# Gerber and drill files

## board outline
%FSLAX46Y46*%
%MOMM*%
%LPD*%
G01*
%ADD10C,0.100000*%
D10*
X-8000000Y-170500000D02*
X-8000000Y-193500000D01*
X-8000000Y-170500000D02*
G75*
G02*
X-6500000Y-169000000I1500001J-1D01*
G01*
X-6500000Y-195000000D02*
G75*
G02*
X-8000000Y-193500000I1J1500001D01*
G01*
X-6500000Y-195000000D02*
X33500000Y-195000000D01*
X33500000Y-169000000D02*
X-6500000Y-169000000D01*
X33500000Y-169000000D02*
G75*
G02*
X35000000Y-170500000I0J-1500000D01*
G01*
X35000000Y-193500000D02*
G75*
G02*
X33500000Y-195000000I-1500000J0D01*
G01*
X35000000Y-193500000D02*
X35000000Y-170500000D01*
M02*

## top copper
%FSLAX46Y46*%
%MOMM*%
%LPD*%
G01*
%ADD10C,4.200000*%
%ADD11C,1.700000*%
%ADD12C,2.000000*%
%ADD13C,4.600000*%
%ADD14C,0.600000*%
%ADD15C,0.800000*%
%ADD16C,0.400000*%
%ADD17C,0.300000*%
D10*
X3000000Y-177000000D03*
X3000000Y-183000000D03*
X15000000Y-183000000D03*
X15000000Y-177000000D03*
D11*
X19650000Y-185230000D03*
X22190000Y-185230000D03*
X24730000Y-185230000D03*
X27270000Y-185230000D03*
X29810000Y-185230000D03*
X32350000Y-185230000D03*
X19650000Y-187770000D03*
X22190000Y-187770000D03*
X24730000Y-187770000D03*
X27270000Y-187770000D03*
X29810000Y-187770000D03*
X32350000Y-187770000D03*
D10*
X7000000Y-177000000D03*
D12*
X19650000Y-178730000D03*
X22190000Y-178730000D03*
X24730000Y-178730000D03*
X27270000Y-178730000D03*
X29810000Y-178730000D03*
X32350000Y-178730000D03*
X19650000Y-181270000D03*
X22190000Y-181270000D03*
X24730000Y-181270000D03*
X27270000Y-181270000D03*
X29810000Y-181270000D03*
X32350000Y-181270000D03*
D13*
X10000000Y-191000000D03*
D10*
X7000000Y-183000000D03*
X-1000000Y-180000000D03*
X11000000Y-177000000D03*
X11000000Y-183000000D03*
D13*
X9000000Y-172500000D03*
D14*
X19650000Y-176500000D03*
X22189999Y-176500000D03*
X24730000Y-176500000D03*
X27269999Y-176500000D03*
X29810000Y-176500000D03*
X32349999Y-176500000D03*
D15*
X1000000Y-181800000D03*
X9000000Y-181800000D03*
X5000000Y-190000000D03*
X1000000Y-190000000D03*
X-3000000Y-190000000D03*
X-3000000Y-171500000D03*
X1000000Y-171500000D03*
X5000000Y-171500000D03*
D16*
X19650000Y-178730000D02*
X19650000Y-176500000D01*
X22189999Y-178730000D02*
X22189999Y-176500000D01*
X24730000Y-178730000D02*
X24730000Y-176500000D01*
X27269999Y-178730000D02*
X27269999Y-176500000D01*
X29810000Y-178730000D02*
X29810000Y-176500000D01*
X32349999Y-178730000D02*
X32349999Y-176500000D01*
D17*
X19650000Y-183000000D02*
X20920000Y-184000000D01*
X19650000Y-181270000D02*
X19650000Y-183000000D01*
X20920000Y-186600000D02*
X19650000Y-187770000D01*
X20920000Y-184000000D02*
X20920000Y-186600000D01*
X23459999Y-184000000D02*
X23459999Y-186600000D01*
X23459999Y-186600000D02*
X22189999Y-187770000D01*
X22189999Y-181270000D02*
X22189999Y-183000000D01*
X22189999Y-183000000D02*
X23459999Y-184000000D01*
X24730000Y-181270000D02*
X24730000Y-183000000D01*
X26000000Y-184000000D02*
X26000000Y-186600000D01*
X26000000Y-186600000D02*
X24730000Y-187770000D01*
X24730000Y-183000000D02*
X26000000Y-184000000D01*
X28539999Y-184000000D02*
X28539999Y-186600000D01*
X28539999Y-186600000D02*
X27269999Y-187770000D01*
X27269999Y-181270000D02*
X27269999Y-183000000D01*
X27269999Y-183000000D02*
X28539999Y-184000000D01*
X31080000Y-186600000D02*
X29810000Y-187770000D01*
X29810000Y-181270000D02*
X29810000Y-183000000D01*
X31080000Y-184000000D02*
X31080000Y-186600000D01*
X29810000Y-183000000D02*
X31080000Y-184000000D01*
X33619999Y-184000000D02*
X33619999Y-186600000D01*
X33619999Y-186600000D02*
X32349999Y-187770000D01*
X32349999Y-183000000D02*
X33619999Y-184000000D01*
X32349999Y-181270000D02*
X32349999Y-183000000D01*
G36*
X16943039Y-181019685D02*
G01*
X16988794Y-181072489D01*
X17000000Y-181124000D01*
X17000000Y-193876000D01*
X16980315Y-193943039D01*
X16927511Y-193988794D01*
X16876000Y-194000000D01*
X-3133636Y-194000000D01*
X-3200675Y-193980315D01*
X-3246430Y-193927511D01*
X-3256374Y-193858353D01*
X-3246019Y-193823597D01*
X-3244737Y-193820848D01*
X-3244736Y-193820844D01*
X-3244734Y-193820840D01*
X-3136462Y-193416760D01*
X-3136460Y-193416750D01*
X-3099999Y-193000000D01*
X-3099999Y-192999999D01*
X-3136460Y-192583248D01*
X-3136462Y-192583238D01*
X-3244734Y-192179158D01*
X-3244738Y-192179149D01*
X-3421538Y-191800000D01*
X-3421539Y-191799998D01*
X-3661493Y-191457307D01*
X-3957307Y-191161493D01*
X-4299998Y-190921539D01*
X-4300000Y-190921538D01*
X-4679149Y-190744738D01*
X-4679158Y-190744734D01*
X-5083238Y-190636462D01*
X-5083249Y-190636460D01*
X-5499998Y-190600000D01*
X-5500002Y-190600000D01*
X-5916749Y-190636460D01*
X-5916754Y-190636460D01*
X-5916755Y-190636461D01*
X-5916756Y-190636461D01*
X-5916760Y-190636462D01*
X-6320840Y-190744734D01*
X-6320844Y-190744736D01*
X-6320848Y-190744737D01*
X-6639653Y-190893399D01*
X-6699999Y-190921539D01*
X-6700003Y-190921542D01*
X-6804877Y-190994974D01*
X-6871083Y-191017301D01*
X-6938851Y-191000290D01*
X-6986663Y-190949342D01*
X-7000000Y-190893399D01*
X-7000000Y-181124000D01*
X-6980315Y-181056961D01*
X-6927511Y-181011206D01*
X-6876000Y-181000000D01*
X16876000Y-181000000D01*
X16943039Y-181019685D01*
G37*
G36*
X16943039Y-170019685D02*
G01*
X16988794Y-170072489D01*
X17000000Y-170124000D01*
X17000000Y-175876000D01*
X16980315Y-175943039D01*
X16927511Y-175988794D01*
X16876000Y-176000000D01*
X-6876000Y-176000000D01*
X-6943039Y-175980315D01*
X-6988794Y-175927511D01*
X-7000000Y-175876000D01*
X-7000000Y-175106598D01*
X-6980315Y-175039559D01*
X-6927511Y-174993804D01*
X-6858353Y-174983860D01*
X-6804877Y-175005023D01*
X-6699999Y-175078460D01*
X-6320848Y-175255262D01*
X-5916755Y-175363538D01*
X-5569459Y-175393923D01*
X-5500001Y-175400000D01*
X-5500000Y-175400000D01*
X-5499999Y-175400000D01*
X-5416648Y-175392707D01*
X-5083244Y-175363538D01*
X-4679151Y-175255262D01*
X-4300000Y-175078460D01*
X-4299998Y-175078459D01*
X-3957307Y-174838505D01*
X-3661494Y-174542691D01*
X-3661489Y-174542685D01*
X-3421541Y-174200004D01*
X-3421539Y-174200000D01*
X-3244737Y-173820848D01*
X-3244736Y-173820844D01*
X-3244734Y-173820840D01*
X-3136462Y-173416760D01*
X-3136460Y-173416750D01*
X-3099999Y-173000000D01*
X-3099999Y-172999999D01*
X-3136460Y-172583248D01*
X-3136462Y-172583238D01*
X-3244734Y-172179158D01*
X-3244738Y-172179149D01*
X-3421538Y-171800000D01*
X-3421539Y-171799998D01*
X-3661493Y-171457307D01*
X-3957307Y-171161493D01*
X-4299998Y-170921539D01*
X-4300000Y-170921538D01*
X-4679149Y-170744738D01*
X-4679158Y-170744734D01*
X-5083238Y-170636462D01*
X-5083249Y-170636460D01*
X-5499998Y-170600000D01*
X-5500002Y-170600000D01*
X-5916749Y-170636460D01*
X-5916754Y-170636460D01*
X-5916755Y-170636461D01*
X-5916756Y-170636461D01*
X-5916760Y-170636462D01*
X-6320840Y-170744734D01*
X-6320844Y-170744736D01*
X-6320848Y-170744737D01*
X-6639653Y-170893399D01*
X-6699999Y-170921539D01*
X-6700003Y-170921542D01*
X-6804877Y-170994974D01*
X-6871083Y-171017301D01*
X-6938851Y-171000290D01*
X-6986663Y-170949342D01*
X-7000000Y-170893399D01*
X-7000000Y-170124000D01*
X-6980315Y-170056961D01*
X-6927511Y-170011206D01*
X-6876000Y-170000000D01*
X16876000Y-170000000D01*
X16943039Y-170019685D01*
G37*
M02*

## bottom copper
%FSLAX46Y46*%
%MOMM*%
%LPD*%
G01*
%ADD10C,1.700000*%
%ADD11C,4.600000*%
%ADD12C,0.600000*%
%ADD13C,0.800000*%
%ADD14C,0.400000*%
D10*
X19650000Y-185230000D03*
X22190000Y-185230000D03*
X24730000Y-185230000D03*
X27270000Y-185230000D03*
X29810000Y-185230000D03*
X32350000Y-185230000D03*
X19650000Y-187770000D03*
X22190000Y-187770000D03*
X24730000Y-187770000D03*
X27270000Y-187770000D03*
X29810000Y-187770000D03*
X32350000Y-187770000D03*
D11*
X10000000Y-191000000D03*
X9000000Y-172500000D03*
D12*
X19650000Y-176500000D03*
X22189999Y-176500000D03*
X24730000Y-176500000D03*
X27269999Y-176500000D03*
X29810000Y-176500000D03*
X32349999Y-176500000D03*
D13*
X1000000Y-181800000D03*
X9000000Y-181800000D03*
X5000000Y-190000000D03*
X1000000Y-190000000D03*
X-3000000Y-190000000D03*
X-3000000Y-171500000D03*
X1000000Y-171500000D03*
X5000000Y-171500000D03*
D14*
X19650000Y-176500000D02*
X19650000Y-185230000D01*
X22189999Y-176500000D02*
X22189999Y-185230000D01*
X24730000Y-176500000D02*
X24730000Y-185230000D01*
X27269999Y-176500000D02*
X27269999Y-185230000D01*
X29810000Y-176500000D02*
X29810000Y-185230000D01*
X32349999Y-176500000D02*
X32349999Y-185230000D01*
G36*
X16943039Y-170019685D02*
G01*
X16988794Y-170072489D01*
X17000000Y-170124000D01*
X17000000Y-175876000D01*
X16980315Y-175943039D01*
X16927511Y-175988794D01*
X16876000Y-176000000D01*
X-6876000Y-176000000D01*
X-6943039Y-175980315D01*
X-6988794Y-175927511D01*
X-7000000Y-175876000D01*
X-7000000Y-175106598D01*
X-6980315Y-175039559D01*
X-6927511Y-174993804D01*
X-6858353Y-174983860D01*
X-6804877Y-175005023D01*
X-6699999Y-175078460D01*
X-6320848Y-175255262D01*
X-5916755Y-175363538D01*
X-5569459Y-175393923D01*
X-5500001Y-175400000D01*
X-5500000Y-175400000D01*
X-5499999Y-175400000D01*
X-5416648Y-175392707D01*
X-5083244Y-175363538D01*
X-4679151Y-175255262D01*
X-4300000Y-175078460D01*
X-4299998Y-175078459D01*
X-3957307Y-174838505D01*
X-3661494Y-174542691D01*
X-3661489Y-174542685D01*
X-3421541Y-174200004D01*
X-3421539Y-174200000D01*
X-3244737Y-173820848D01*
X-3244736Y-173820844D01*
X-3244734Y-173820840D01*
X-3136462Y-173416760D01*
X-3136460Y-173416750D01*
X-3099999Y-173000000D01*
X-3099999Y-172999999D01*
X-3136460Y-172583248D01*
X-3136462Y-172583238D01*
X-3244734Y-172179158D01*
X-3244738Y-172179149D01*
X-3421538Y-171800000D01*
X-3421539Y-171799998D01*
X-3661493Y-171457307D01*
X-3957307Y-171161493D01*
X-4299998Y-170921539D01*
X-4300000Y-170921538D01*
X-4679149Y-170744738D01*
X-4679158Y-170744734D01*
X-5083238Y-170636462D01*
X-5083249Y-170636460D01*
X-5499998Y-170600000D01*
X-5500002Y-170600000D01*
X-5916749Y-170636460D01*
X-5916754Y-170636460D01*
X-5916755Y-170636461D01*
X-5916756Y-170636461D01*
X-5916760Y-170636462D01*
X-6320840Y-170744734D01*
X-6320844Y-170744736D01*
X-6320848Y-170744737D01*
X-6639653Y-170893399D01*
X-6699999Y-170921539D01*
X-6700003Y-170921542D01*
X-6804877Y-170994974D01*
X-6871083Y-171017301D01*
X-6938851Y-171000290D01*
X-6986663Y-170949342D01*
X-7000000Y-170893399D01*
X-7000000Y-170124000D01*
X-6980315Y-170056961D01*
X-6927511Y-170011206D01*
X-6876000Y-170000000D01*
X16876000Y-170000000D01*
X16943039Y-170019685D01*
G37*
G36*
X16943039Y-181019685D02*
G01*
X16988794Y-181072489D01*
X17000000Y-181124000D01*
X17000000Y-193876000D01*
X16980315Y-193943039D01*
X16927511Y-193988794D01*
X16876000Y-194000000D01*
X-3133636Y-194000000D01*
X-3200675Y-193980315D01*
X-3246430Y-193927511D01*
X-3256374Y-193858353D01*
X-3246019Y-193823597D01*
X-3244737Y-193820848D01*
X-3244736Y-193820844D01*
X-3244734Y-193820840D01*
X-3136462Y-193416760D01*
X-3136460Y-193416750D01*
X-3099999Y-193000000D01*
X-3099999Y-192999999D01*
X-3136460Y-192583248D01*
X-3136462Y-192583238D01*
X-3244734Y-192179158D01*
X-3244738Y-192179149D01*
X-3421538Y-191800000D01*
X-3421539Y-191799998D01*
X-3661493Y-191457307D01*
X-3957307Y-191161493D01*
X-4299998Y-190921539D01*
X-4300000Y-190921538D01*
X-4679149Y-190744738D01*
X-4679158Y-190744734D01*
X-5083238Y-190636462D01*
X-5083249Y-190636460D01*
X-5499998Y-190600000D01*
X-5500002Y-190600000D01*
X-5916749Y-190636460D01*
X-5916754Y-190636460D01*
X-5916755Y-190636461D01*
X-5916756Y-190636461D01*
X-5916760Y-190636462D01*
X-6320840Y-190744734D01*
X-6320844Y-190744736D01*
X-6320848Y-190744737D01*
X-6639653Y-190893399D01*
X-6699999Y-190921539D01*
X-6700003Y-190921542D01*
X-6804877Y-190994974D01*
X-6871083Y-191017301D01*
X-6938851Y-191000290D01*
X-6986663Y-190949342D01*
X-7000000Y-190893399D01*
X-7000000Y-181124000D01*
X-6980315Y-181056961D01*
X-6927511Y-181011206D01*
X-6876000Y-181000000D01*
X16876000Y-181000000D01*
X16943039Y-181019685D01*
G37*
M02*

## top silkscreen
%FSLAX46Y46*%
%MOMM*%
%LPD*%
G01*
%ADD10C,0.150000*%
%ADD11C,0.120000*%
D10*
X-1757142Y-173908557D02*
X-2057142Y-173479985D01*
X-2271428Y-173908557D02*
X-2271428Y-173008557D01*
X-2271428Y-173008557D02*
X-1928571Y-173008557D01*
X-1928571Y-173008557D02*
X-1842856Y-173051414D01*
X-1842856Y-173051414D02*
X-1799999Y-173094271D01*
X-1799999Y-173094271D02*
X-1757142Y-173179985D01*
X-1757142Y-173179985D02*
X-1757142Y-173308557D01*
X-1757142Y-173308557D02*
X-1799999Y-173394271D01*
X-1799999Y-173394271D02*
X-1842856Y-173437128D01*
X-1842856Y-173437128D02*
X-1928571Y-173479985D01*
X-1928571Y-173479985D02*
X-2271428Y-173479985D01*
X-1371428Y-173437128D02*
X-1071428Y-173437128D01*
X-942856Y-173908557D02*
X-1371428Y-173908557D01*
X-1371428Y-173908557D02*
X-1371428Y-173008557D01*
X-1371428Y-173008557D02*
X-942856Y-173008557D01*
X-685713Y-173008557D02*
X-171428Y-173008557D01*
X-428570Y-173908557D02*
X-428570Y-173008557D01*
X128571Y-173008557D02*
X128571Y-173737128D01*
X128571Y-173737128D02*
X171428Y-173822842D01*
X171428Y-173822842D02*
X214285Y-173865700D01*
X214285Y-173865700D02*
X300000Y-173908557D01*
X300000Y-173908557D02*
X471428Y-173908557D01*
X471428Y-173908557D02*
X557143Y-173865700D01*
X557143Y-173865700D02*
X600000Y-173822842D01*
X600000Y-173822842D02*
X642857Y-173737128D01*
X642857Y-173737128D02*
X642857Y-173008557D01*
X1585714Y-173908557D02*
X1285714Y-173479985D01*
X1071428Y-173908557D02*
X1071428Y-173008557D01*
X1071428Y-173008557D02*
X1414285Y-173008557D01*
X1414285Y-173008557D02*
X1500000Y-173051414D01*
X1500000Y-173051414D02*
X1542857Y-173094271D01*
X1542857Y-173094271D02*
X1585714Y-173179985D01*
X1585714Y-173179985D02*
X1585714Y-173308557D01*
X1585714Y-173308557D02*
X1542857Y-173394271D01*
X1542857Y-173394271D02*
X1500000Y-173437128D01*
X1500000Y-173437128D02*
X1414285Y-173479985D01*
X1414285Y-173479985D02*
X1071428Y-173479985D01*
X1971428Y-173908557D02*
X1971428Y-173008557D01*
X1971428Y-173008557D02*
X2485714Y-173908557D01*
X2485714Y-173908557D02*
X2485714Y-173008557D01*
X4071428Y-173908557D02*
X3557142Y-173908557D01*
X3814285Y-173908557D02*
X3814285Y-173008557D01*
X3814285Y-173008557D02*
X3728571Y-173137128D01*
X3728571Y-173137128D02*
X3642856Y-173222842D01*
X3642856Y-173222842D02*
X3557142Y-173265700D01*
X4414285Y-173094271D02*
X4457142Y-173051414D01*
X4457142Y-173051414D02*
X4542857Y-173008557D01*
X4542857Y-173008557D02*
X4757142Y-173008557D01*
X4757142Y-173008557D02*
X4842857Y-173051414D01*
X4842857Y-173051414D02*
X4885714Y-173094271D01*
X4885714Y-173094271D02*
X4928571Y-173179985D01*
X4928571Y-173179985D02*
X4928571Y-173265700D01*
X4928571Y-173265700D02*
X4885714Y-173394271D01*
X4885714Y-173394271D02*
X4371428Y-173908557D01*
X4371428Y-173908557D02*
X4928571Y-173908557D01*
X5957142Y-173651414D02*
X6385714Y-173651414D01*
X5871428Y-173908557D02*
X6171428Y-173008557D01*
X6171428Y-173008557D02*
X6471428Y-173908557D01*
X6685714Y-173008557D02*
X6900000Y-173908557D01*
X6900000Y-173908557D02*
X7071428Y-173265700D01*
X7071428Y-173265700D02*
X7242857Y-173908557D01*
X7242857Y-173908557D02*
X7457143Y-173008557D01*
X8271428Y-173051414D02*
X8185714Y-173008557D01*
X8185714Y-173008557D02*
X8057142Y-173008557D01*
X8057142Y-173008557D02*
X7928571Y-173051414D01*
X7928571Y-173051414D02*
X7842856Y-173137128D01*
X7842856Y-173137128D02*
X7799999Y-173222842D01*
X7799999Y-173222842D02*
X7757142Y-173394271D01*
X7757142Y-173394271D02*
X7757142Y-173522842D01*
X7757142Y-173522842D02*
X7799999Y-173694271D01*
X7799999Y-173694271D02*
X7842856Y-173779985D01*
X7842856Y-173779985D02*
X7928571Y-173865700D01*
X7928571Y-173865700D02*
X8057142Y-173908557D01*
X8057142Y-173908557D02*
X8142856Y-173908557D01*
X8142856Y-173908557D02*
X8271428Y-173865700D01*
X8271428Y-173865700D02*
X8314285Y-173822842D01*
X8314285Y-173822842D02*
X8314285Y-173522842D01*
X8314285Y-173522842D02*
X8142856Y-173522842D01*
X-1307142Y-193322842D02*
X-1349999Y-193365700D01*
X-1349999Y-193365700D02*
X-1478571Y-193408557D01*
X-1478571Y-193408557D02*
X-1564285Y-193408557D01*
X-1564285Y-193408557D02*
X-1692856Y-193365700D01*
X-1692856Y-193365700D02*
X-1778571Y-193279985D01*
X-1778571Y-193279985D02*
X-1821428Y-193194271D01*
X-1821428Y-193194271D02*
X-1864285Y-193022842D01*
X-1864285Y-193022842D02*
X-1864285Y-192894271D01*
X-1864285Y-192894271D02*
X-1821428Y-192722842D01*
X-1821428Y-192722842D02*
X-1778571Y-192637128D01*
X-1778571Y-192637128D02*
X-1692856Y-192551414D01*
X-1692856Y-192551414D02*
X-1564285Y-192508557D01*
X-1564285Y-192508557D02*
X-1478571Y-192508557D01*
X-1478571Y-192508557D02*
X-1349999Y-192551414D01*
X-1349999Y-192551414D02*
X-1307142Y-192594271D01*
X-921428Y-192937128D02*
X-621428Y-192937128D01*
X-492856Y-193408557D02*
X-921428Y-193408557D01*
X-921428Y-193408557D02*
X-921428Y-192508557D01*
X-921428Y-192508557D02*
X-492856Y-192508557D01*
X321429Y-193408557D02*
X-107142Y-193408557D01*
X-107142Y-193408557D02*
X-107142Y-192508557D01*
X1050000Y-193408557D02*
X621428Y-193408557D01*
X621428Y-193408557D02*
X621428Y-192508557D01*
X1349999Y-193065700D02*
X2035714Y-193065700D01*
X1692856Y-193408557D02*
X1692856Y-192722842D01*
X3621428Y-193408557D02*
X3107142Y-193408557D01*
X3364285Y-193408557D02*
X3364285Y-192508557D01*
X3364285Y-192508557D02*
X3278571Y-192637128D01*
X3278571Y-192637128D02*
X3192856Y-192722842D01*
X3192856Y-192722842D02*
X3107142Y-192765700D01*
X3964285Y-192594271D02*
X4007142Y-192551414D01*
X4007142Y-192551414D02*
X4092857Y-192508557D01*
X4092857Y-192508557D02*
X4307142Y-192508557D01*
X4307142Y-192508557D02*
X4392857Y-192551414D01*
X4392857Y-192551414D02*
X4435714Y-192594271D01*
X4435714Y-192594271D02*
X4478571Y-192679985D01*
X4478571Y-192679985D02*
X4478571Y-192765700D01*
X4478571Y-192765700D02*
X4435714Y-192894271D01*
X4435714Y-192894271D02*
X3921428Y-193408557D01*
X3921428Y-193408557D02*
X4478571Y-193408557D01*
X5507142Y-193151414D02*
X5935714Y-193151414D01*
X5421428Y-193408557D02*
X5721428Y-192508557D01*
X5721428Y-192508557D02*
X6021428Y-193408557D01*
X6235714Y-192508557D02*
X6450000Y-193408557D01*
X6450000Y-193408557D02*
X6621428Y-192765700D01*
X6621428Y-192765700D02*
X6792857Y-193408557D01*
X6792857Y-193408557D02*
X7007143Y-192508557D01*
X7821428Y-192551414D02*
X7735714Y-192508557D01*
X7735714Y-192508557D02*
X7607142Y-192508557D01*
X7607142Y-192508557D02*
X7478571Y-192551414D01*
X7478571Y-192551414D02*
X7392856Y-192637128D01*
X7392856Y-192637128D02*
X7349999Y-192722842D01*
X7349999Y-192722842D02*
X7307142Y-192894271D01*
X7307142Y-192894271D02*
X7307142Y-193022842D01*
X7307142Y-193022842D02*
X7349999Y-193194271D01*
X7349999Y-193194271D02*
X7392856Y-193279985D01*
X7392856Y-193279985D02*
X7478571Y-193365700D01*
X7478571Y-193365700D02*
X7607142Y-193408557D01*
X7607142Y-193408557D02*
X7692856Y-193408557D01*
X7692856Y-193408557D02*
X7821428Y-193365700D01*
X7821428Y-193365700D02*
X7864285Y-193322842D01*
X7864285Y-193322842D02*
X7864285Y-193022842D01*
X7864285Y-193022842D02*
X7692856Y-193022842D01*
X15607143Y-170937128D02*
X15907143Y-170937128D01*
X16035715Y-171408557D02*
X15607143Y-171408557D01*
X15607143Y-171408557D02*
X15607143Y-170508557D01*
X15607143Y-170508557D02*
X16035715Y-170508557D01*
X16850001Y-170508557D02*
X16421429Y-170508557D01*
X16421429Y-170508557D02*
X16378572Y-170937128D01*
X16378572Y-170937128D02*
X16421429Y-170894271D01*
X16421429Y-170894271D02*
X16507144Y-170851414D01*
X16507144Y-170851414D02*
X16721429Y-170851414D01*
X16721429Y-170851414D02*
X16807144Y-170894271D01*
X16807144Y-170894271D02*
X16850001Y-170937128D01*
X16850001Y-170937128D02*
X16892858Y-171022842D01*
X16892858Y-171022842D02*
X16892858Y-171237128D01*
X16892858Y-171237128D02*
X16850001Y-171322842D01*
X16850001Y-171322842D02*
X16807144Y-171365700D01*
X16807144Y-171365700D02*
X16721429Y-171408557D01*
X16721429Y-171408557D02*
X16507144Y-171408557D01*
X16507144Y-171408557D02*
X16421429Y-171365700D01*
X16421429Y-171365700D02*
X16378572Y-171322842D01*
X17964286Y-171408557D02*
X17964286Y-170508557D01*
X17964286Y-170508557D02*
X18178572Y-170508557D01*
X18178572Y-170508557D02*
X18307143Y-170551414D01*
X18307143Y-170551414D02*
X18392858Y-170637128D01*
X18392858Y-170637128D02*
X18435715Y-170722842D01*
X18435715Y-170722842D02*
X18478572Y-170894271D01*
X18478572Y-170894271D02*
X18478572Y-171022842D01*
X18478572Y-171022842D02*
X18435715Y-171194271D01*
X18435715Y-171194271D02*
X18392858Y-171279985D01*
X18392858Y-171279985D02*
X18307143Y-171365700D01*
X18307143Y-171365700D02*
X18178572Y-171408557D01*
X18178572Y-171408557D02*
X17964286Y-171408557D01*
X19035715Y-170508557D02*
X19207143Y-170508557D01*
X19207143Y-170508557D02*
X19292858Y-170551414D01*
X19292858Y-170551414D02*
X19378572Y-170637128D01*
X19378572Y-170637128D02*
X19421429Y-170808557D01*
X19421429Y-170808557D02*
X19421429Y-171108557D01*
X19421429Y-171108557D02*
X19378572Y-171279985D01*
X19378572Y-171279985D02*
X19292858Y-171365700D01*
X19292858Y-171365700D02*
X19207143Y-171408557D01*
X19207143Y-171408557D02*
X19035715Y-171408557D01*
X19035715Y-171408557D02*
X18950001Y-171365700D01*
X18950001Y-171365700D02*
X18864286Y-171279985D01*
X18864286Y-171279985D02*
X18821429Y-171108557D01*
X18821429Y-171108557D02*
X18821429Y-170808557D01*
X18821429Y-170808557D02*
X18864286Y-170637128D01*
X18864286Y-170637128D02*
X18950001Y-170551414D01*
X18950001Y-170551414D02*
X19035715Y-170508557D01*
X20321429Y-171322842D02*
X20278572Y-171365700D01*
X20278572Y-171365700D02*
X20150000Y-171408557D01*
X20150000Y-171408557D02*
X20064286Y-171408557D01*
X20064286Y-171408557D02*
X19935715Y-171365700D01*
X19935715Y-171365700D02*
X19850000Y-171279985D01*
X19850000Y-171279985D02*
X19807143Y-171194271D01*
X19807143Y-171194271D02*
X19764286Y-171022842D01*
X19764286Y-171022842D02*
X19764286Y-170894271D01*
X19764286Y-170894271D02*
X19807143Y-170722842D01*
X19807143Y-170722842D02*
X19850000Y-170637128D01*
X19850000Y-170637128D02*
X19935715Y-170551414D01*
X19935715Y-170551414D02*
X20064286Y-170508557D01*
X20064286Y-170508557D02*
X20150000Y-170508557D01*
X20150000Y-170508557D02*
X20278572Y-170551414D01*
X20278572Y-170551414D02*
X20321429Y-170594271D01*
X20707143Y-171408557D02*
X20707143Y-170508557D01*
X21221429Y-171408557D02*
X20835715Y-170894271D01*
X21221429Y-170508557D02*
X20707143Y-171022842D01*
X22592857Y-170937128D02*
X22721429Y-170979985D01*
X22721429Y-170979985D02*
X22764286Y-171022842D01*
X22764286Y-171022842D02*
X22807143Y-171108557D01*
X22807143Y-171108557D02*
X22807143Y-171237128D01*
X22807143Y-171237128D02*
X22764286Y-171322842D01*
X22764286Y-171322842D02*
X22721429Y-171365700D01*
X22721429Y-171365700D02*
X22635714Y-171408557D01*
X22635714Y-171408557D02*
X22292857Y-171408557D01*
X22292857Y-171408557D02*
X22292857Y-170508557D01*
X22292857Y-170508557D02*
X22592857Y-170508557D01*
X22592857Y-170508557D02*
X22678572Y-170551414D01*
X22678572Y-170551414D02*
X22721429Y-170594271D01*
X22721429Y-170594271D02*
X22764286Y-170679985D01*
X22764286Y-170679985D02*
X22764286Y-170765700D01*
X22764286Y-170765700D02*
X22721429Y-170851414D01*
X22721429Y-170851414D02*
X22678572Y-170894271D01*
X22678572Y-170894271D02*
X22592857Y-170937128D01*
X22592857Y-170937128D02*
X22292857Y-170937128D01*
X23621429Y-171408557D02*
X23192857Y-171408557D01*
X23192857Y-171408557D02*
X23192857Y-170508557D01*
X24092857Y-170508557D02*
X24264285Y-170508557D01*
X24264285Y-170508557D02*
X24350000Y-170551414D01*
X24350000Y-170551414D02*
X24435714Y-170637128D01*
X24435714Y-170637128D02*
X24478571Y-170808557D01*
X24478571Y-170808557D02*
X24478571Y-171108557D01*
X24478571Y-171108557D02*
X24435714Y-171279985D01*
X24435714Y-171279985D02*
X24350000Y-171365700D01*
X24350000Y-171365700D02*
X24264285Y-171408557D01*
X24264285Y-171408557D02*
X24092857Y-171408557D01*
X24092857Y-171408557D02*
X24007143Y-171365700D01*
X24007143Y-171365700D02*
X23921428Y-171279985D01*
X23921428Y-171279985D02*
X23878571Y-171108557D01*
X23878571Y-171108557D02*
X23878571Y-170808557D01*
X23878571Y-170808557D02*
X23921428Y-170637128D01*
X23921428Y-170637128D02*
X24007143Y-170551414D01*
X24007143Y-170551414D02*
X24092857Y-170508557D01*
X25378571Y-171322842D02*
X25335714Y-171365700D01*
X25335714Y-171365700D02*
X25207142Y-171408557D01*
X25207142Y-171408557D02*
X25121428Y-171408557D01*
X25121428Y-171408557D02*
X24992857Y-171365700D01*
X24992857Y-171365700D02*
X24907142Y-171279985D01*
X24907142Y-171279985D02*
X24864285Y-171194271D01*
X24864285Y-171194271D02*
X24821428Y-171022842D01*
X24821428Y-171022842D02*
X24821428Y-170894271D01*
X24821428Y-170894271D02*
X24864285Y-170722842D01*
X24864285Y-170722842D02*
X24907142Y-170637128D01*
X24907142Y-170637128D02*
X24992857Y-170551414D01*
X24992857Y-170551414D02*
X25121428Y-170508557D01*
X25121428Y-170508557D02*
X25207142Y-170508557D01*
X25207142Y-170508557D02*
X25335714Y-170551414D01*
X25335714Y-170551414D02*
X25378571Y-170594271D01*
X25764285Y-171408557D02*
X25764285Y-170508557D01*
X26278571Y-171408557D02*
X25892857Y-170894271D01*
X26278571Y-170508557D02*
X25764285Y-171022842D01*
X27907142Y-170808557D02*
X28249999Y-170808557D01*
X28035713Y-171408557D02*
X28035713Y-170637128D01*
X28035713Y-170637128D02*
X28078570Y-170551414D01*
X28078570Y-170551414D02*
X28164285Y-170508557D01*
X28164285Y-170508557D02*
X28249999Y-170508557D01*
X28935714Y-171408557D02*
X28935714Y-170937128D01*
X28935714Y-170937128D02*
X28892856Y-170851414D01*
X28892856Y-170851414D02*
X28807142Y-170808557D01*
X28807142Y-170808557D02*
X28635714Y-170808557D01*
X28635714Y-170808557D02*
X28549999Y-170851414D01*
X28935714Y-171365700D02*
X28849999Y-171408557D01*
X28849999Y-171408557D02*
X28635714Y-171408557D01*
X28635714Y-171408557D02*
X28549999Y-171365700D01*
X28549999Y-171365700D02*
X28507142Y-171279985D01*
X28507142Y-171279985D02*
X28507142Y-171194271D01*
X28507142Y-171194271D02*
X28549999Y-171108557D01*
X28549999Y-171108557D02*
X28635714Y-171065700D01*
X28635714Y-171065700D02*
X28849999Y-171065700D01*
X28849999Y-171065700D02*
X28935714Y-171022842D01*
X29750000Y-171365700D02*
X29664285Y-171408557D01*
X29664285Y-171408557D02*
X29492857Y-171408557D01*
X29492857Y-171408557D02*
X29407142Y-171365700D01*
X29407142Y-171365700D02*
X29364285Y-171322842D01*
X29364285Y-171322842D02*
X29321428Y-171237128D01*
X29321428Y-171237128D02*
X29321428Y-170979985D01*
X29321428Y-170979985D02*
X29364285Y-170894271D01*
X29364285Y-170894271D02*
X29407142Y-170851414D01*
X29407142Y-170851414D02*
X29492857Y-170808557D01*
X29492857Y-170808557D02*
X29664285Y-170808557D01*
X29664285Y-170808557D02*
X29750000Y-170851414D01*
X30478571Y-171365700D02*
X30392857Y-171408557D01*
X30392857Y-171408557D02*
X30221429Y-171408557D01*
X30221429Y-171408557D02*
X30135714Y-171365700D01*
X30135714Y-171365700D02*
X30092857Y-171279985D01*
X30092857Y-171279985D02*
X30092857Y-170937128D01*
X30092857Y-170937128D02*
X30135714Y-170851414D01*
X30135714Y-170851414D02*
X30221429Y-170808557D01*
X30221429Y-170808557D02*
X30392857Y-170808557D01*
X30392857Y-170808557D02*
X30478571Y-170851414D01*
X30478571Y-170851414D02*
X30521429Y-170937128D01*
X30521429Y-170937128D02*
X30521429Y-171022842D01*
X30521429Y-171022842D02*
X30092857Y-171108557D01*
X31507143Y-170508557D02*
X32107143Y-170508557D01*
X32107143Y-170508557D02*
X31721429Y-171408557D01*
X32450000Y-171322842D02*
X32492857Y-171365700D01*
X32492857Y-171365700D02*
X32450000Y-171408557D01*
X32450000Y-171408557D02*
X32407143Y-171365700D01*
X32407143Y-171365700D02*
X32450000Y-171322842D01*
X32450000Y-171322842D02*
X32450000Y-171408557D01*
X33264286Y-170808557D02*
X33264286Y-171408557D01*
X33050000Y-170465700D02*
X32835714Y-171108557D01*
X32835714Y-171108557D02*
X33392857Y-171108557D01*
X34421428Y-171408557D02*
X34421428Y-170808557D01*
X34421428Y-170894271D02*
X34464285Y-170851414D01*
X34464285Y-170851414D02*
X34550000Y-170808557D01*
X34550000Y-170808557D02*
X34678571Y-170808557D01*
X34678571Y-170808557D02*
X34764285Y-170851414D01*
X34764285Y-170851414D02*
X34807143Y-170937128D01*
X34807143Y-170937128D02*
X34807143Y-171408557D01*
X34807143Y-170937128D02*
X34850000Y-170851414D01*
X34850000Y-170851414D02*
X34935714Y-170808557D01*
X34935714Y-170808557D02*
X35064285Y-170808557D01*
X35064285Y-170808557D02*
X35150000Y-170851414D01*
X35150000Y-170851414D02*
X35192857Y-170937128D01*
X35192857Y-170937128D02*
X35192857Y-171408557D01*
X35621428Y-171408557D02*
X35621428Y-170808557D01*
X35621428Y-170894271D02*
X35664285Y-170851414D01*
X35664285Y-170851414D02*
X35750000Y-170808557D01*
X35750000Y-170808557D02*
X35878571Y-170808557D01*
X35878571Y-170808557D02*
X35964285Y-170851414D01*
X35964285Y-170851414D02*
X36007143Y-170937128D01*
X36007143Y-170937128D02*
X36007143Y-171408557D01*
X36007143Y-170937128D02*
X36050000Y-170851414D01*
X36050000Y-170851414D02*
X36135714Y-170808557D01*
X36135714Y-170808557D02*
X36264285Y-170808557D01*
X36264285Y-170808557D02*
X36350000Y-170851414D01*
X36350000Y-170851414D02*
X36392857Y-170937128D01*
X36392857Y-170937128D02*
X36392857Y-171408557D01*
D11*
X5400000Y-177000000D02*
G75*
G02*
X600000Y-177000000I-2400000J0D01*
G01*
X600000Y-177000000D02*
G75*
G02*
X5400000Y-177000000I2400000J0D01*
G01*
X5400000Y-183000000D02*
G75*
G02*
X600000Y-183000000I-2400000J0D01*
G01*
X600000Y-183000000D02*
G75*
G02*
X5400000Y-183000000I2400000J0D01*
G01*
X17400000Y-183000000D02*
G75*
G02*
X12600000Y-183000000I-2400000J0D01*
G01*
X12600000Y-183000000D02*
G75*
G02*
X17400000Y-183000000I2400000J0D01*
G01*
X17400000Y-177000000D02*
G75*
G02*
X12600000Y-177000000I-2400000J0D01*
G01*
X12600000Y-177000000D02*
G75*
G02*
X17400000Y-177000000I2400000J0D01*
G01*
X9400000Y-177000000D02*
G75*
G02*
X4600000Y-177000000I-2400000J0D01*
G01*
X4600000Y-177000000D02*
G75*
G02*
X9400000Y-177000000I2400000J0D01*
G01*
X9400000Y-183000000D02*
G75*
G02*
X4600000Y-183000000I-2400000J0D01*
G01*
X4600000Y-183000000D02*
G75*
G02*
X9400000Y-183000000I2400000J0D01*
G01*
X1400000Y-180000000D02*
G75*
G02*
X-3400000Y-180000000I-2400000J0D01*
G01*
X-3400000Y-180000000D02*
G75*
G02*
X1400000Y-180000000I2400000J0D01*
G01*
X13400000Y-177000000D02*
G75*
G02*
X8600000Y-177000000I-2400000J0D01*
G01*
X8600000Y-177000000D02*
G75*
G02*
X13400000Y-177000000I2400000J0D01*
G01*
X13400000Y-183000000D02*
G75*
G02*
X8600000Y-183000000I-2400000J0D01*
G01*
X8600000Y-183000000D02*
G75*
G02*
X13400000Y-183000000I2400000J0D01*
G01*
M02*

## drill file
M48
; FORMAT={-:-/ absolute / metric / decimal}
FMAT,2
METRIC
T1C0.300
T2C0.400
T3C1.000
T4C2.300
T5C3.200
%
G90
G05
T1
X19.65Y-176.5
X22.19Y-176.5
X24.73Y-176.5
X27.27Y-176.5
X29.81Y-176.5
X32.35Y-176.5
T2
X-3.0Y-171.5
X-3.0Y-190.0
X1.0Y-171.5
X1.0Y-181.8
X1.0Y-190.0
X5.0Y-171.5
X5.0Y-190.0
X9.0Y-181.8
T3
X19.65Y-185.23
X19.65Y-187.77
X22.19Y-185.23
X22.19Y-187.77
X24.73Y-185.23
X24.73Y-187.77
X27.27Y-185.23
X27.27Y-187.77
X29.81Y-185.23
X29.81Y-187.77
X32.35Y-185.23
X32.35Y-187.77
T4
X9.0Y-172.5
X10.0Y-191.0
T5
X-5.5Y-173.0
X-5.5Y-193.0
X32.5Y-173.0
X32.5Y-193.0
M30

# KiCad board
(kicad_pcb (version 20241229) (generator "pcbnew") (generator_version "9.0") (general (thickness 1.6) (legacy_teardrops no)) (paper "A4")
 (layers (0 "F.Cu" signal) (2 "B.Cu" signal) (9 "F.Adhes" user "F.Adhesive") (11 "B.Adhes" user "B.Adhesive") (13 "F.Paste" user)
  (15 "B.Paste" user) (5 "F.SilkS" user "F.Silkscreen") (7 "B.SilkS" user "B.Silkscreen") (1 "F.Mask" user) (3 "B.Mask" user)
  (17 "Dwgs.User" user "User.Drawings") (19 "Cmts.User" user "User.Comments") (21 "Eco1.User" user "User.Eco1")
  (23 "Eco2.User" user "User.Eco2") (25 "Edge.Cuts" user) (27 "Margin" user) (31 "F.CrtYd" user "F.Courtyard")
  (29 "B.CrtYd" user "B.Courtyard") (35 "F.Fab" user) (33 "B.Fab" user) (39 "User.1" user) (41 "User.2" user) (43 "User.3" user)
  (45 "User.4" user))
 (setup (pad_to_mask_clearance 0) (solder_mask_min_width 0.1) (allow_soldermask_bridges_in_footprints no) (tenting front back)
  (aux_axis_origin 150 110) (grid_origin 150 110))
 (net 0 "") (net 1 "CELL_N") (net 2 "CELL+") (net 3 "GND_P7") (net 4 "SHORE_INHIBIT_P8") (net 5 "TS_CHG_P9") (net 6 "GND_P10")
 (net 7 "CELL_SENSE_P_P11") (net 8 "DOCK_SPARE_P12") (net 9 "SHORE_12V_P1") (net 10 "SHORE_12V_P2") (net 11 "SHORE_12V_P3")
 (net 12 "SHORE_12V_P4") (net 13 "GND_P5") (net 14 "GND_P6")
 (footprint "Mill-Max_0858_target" (layer "F.Cu") (at 3 177)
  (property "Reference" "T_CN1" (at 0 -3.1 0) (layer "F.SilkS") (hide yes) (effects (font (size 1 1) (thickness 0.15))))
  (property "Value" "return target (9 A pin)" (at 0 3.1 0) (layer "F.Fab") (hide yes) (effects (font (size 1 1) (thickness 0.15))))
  (fp_circle (center 0 0) (end 2.4 0) (stroke (width 0.12) (type solid)) (fill no) (layer "F.SilkS"))
  (pad "1" smd circle (at 0 0) (size 4.2 4.2) (layers "F.Cu" "F.Mask") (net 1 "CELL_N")))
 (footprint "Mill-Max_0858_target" (layer "F.Cu") (at 3 183)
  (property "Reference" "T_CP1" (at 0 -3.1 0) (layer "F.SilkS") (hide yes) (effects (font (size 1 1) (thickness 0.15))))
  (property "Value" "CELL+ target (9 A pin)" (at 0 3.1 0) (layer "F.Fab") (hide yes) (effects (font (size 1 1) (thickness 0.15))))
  (fp_circle (center 0 0) (end 2.4 0) (stroke (width 0.12) (type solid)) (fill no) (layer "F.SilkS"))
  (pad "1" smd circle (at 0 0) (size 4.2 4.2) (layers "F.Cu" "F.Mask") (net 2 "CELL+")))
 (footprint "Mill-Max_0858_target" (layer "F.Cu") (at 15 183)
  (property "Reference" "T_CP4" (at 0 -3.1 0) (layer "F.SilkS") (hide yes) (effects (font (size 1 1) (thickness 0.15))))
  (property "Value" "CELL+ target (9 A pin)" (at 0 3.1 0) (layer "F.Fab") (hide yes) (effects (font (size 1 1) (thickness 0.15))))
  (fp_circle (center 0 0) (end 2.4 0) (stroke (width 0.12) (type solid)) (fill no) (layer "F.SilkS"))
  (pad "1" smd circle (at 0 0) (size 4.2 4.2) (layers "F.Cu" "F.Mask") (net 2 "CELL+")))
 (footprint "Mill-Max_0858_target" (layer "F.Cu") (at 15 177)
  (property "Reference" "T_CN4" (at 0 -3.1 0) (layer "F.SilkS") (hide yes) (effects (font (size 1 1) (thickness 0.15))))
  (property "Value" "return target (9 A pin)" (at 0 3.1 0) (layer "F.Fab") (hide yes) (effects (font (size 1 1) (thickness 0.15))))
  (fp_circle (center 0 0) (end 2.4 0) (stroke (width 0.12) (type solid)) (fill no) (layer "F.SilkS"))
  (pad "1" smd circle (at 0 0) (size 4.2 4.2) (layers "F.Cu" "F.Mask") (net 1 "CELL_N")))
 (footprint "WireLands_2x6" (layer "F.Cu") (at 26 186.5)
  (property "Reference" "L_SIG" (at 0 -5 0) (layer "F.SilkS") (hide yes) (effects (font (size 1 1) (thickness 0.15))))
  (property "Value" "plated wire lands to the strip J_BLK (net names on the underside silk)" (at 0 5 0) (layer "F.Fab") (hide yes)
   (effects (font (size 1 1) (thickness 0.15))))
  (pad "1" thru_hole circle (at -6.35 -1.27) (size 1.7 1.7) (drill 1) (layers "*.Cu" "*.Mask") (remove_unused_layers no) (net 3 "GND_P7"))
  (pad "2" thru_hole circle (at -3.81 -1.27) (size 1.7 1.7) (drill 1) (layers "*.Cu" "*.Mask") (remove_unused_layers no)
   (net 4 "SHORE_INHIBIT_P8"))
  (pad "3" thru_hole circle (at -1.27 -1.27) (size 1.7 1.7) (drill 1) (layers "*.Cu" "*.Mask") (remove_unused_layers no) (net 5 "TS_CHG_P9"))
  (pad "4" thru_hole circle (at 1.27 -1.27) (size 1.7 1.7) (drill 1) (layers "*.Cu" "*.Mask") (remove_unused_layers no) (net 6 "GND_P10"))
  (pad "5" thru_hole circle (at 3.81 -1.27) (size 1.7 1.7) (drill 1) (layers "*.Cu" "*.Mask") (remove_unused_layers no)
   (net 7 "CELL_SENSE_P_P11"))
  (pad "6" thru_hole circle (at 6.35 -1.27) (size 1.7 1.7) (drill 1) (layers "*.Cu" "*.Mask") (remove_unused_layers no)
   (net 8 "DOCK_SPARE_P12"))
  (pad "7" thru_hole circle (at -6.35 1.27) (size 1.7 1.7) (drill 1) (layers "*.Cu" "*.Mask") (remove_unused_layers no)
   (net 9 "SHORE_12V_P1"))
  (pad "8" thru_hole circle (at -3.81 1.27) (size 1.7 1.7) (drill 1) (layers "*.Cu" "*.Mask") (remove_unused_layers no)
   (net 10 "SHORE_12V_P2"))
  (pad "9" thru_hole circle (at -1.27 1.27) (size 1.7 1.7) (drill 1) (layers "*.Cu" "*.Mask") (remove_unused_layers no)
   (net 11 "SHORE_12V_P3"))
  (pad "10" thru_hole circle (at 1.27 1.27) (size 1.7 1.7) (drill 1) (layers "*.Cu" "*.Mask") (remove_unused_layers no)
   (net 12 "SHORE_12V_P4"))
  (pad "11" thru_hole circle (at 3.81 1.27) (size 1.7 1.7) (drill 1) (layers "*.Cu" "*.Mask") (remove_unused_layers no) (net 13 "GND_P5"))
  (pad "12" thru_hole circle (at 6.35 1.27) (size 1.7 1.7) (drill 1) (layers "*.Cu" "*.Mask") (remove_unused_layers no) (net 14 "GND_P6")))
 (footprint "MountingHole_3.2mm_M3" (layer "F.Cu") (at -5.5 173)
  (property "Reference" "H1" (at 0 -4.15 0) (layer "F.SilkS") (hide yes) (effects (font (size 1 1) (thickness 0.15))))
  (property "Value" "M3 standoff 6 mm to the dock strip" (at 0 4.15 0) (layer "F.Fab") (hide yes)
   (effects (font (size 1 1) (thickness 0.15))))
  (pad "" np_thru_hole circle (at 0 0) (size 3.2 3.2) (drill 3.2) (layers "*.Cu" "*.Mask")))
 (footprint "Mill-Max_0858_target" (layer "F.Cu") (at 7 177)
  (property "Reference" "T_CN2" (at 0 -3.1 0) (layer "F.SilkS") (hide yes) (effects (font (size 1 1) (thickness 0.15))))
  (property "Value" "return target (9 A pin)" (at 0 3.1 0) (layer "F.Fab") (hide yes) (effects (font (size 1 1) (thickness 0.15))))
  (fp_circle (center 0 0) (end 2.4 0) (stroke (width 0.12) (type solid)) (fill no) (layer "F.SilkS"))
  (pad "1" smd circle (at 0 0) (size 4.2 4.2) (layers "F.Cu" "F.Mask") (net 1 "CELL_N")))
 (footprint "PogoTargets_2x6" (layer "F.Cu") (at 26 180)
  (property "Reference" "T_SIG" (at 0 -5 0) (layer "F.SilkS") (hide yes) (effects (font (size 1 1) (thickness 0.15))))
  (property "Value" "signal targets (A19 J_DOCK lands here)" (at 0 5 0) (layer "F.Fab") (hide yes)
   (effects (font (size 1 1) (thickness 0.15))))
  (pad "1" smd circle (at -6.35 -1.27) (size 2 2) (layers "F.Cu" "F.Mask") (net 3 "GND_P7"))
  (pad "2" smd circle (at -3.81 -1.27) (size 2 2) (layers "F.Cu" "F.Mask") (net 4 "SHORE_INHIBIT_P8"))
  (pad "3" smd circle (at -1.27 -1.27) (size 2 2) (layers "F.Cu" "F.Mask") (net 5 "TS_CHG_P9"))
  (pad "4" smd circle (at 1.27 -1.27) (size 2 2) (layers "F.Cu" "F.Mask") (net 6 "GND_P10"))
  (pad "5" smd circle (at 3.81 -1.27) (size 2 2) (layers "F.Cu" "F.Mask") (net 7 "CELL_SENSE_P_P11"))
  (pad "6" smd circle (at 6.35 -1.27) (size 2 2) (layers "F.Cu" "F.Mask") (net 8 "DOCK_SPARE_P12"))
  (pad "7" smd circle (at -6.35 1.27) (size 2 2) (layers "F.Cu" "F.Mask") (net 9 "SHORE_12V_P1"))
  (pad "8" smd circle (at -3.81 1.27) (size 2 2) (layers "F.Cu" "F.Mask") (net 10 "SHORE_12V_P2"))
  (pad "9" smd circle (at -1.27 1.27) (size 2 2) (layers "F.Cu" "F.Mask") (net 11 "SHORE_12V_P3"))
  (pad "10" smd circle (at 1.27 1.27) (size 2 2) (layers "F.Cu" "F.Mask") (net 12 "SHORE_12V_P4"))
  (pad "11" smd circle (at 3.81 1.27) (size 2 2) (layers "F.Cu" "F.Mask") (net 13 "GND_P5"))
  (pad "12" smd circle (at 6.35 1.27) (size 2 2) (layers "F.Cu" "F.Mask") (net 14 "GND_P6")))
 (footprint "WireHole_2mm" (layer "F.Cu") (at 10 191)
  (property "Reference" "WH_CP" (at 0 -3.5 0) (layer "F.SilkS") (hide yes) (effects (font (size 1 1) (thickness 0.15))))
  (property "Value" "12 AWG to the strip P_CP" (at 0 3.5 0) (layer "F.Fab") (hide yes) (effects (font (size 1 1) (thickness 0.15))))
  (pad "1" thru_hole circle (at 0 0) (size 4.6 4.6) (drill 2.3) (layers "*.Cu" "*.Mask") (remove_unused_layers no) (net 2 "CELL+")))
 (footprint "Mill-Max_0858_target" (layer "F.Cu") (at 7 183)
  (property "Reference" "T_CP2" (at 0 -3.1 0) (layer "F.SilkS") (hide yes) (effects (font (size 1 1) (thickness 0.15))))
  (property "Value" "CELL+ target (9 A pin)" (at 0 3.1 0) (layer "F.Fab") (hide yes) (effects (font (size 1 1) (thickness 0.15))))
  (fp_circle (center 0 0) (end 2.4 0) (stroke (width 0.12) (type solid)) (fill no) (layer "F.SilkS"))
  (pad "1" smd circle (at 0 0) (size 4.2 4.2) (layers "F.Cu" "F.Mask") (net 2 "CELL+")))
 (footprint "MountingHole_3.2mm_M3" (layer "F.Cu") (at 32.5 173)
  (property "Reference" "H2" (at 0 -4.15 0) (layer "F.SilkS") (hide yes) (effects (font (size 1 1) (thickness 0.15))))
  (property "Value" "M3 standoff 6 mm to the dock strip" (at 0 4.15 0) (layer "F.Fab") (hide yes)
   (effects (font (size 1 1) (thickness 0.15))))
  (pad "" np_thru_hole circle (at 0 0) (size 3.2 3.2) (drill 3.2) (layers "*.Cu" "*.Mask")))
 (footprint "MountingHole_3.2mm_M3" (layer "F.Cu") (at -5.5 193)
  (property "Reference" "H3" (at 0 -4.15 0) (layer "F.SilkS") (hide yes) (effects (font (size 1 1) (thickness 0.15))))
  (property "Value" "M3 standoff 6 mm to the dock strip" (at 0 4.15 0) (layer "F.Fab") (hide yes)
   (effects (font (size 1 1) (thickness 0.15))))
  (pad "" np_thru_hole circle (at 0 0) (size 3.2 3.2) (drill 3.2) (layers "*.Cu" "*.Mask")))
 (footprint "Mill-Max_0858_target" (layer "F.Cu") (at -1 180)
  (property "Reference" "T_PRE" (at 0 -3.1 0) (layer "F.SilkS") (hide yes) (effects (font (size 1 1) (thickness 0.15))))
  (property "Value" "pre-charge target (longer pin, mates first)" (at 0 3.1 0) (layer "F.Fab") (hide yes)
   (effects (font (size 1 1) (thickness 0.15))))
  (fp_circle (center 0 0) (end 2.4 0) (stroke (width 0.12) (type solid)) (fill no) (layer "F.SilkS"))
  (pad "1" smd circle (at 0 0) (size 4.2 4.2) (layers "F.Cu" "F.Mask") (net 2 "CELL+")))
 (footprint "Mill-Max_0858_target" (layer "F.Cu") (at 11 177)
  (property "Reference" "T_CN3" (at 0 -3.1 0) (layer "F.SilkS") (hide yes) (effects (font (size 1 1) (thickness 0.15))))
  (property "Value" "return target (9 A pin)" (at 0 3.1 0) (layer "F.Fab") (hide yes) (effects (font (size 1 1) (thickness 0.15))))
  (fp_circle (center 0 0) (end 2.4 0) (stroke (width 0.12) (type solid)) (fill no) (layer "F.SilkS"))
  (pad "1" smd circle (at 0 0) (size 4.2 4.2) (layers "F.Cu" "F.Mask") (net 1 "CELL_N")))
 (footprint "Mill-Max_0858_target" (layer "F.Cu") (at 11 183)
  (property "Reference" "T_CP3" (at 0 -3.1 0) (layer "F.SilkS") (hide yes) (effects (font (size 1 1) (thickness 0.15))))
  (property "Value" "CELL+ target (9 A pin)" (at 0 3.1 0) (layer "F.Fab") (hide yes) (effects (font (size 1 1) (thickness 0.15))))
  (fp_circle (center 0 0) (end 2.4 0) (stroke (width 0.12) (type solid)) (fill no) (layer "F.SilkS"))
  (pad "1" smd circle (at 0 0) (size 4.2 4.2) (layers "F.Cu" "F.Mask") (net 2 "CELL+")))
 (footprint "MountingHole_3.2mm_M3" (layer "F.Cu") (at 32.5 193)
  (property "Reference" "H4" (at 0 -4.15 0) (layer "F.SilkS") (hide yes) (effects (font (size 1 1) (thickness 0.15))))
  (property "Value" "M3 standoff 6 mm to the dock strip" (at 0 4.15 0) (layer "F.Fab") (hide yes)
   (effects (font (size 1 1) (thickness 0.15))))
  (pad "" np_thru_hole circle (at 0 0) (size 3.2 3.2) (drill 3.2) (layers "*.Cu" "*.Mask")))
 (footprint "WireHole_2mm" (layer "F.Cu") (at 9 172.5)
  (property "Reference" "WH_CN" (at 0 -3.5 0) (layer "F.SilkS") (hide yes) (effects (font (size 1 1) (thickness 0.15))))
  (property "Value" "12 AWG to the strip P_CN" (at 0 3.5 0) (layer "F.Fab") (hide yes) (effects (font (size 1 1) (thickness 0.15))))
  (pad "1" thru_hole circle (at 0 0) (size 4.6 4.6) (drill 2.3) (layers "*.Cu" "*.Mask") (remove_unused_layers no) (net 1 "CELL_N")))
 (gr_line (start -8 170.5) (end -8 193.5) (stroke (width 0.1) (type default)) (layer "Edge.Cuts"))
 (gr_arc (start -8 170.5) (mid -7.56066 169.43934) (end -6.5 169) (stroke (width 0.1) (type default)) (layer "Edge.Cuts"))
 (gr_arc (start -6.5 195) (mid -7.56066 194.56066) (end -8 193.5) (stroke (width 0.1) (type default)) (layer "Edge.Cuts"))
 (gr_line (start -6.5 195) (end 33.5 195) (stroke (width 0.1) (type default)) (layer "Edge.Cuts"))
 (gr_line (start 33.5 169) (end -6.5 169) (stroke (width 0.1) (type default)) (layer "Edge.Cuts"))
 (gr_arc (start 33.5 169) (mid 34.56066 169.43934) (end 35 170.5) (stroke (width 0.1) (type default)) (layer "Edge.Cuts"))
 (gr_arc (start 35 193.5) (mid 34.56066 194.56066) (end 33.5 195) (stroke (width 0.1) (type default)) (layer "Edge.Cuts"))
 (gr_line (start 35 193.5) (end 35 170.5) (stroke (width 0.1) (type default)) (layer "Edge.Cuts"))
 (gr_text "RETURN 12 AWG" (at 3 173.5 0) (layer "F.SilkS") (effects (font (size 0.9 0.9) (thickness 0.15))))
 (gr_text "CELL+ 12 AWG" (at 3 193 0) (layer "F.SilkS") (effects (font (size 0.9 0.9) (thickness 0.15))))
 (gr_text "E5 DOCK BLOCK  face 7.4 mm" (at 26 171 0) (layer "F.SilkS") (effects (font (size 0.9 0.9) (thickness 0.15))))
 (segment (start 19.65 178.73) (end 19.65 176.5) (width 0.4) (layer "F.Cu") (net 3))
 (via (at 19.65 176.5) (size 0.6) (drill 0.3) (layers "F.Cu" "B.Cu") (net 3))
 (segment (start 19.65 176.5) (end 19.65 185.23) (width 0.4) (layer "B.Cu") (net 3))
 (segment (start 22.189999 178.73) (end 22.189999 176.5) (width 0.4) (layer "F.Cu") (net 4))
 (via (at 22.189999 176.5) (size 0.6) (drill 0.3) (layers "F.Cu" "B.Cu") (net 4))
 (segment (start 22.189999 176.5) (end 22.189999 185.23) (width 0.4) (layer "B.Cu") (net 4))
 (segment (start 24.73 178.73) (end 24.73 176.5) (width 0.4) (layer "F.Cu") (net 5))
 (via (at 24.73 176.5) (size 0.6) (drill 0.3) (layers "F.Cu" "B.Cu") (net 5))
 (segment (start 24.73 176.5) (end 24.73 185.23) (width 0.4) (layer "B.Cu") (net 5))
 (segment (start 27.269999 178.73) (end 27.269999 176.5) (width 0.4) (layer "F.Cu") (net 6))
 (via (at 27.269999 176.5) (size 0.6) (drill 0.3) (layers "F.Cu" "B.Cu") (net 6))
 (segment (start 27.269999 176.5) (end 27.269999 185.23) (width 0.4) (layer "B.Cu") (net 6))
 (segment (start 29.81 178.73) (end 29.81 176.5) (width 0.4) (layer "F.Cu") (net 7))
 (via (at 29.81 176.5) (size 0.6) (drill 0.3) (layers "F.Cu" "B.Cu") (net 7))
 (segment (start 29.81 176.5) (end 29.81 185.23) (width 0.4) (layer "B.Cu") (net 7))
 (segment (start 32.349999 178.73) (end 32.349999 176.5) (width 0.4) (layer "F.Cu") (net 8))
 (via (at 32.349999 176.5) (size 0.6) (drill 0.3) (layers "F.Cu" "B.Cu") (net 8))
 (segment (start 32.349999 176.5) (end 32.349999 185.23) (width 0.4) (layer "B.Cu") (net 8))
 (segment (start 19.65 183) (end 20.92 184) (width 0.3) (layer "F.Cu") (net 9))
 (segment (start 19.65 181.27) (end 19.65 183) (width 0.3) (layer "F.Cu") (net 9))
 (segment (start 20.92 186.6) (end 19.65 187.77) (width 0.3) (layer "F.Cu") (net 9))
 (segment (start 20.92 184) (end 20.92 186.6) (width 0.3) (layer "F.Cu") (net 9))
 (segment (start 23.459999 184) (end 23.459999 186.6) (width 0.3) (layer "F.Cu") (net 10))
 (segment (start 23.459999 186.6) (end 22.189999 187.77) (width 0.3) (layer "F.Cu") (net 10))
 (segment (start 22.189999 181.27) (end 22.189999 183) (width 0.3) (layer "F.Cu") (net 10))
 (segment (start 22.189999 183) (end 23.459999 184) (width 0.3) (layer "F.Cu") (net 10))
 (segment (start 24.73 181.27) (end 24.73 183) (width 0.3) (layer "F.Cu") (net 11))
 (segment (start 26 184) (end 26 186.6) (width 0.3) (layer "F.Cu") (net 11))
 (segment (start 26 186.6) (end 24.73 187.77) (width 0.3) (layer "F.Cu") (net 11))
 (segment (start 24.73 183) (end 26 184) (width 0.3) (layer "F.Cu") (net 11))
 (segment (start 28.539999 184) (end 28.539999 186.6) (width 0.3) (layer "F.Cu") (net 12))
 (segment (start 28.539999 186.6) (end 27.269999 187.77) (width 0.3) (layer "F.Cu") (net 12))
 (segment (start 27.269999 181.27) (end 27.269999 183) (width 0.3) (layer "F.Cu") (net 12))
 (segment (start 27.269999 183) (end 28.539999 184) (width 0.3) (layer "F.Cu") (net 12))
 (segment (start 31.08 186.6) (end 29.81 187.77) (width 0.3) (layer "F.Cu") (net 13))
 (segment (start 29.81 181.27) (end 29.81 183) (width 0.3) (layer "F.Cu") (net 13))
 (segment (start 31.08 184) (end 31.08 186.6) (width 0.3) (layer "F.Cu") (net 13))
 (segment (start 29.81 183) (end 31.08 184) (width 0.3) (layer "F.Cu") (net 13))
 (segment (start 33.619999 184) (end 33.619999 186.6) (width 0.3) (layer "F.Cu") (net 14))
 (segment (start 33.619999 186.6) (end 32.349999 187.77) (width 0.3) (layer "F.Cu") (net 14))
 (segment (start 32.349999 183) (end 33.619999 184) (width 0.3) (layer "F.Cu") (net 14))
 (segment (start 32.349999 181.27) (end 32.349999 183) (width 0.3) (layer "F.Cu") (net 14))
 (via (at 1 181.8) (size 0.8) (drill 0.4) (layers "F.Cu" "B.Cu") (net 2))
 (via (at 9 181.8) (size 0.8) (drill 0.4) (layers "F.Cu" "B.Cu") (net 2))
 (via (at 5 190) (size 0.8) (drill 0.4) (layers "F.Cu" "B.Cu") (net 2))
 (via (at 1 190) (size 0.8) (drill 0.4) (layers "F.Cu" "B.Cu") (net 2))
 (via (at -3 190) (size 0.8) (drill 0.4) (layers "F.Cu" "B.Cu") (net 2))
 (via (at -3 171.5) (size 0.8) (drill 0.4) (layers "F.Cu" "B.Cu") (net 1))
 (via (at 1 171.5) (size 0.8) (drill 0.4) (layers "F.Cu" "B.Cu") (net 1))
 (via (at 5 171.5) (size 0.8) (drill 0.4) (layers "F.Cu" "B.Cu") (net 1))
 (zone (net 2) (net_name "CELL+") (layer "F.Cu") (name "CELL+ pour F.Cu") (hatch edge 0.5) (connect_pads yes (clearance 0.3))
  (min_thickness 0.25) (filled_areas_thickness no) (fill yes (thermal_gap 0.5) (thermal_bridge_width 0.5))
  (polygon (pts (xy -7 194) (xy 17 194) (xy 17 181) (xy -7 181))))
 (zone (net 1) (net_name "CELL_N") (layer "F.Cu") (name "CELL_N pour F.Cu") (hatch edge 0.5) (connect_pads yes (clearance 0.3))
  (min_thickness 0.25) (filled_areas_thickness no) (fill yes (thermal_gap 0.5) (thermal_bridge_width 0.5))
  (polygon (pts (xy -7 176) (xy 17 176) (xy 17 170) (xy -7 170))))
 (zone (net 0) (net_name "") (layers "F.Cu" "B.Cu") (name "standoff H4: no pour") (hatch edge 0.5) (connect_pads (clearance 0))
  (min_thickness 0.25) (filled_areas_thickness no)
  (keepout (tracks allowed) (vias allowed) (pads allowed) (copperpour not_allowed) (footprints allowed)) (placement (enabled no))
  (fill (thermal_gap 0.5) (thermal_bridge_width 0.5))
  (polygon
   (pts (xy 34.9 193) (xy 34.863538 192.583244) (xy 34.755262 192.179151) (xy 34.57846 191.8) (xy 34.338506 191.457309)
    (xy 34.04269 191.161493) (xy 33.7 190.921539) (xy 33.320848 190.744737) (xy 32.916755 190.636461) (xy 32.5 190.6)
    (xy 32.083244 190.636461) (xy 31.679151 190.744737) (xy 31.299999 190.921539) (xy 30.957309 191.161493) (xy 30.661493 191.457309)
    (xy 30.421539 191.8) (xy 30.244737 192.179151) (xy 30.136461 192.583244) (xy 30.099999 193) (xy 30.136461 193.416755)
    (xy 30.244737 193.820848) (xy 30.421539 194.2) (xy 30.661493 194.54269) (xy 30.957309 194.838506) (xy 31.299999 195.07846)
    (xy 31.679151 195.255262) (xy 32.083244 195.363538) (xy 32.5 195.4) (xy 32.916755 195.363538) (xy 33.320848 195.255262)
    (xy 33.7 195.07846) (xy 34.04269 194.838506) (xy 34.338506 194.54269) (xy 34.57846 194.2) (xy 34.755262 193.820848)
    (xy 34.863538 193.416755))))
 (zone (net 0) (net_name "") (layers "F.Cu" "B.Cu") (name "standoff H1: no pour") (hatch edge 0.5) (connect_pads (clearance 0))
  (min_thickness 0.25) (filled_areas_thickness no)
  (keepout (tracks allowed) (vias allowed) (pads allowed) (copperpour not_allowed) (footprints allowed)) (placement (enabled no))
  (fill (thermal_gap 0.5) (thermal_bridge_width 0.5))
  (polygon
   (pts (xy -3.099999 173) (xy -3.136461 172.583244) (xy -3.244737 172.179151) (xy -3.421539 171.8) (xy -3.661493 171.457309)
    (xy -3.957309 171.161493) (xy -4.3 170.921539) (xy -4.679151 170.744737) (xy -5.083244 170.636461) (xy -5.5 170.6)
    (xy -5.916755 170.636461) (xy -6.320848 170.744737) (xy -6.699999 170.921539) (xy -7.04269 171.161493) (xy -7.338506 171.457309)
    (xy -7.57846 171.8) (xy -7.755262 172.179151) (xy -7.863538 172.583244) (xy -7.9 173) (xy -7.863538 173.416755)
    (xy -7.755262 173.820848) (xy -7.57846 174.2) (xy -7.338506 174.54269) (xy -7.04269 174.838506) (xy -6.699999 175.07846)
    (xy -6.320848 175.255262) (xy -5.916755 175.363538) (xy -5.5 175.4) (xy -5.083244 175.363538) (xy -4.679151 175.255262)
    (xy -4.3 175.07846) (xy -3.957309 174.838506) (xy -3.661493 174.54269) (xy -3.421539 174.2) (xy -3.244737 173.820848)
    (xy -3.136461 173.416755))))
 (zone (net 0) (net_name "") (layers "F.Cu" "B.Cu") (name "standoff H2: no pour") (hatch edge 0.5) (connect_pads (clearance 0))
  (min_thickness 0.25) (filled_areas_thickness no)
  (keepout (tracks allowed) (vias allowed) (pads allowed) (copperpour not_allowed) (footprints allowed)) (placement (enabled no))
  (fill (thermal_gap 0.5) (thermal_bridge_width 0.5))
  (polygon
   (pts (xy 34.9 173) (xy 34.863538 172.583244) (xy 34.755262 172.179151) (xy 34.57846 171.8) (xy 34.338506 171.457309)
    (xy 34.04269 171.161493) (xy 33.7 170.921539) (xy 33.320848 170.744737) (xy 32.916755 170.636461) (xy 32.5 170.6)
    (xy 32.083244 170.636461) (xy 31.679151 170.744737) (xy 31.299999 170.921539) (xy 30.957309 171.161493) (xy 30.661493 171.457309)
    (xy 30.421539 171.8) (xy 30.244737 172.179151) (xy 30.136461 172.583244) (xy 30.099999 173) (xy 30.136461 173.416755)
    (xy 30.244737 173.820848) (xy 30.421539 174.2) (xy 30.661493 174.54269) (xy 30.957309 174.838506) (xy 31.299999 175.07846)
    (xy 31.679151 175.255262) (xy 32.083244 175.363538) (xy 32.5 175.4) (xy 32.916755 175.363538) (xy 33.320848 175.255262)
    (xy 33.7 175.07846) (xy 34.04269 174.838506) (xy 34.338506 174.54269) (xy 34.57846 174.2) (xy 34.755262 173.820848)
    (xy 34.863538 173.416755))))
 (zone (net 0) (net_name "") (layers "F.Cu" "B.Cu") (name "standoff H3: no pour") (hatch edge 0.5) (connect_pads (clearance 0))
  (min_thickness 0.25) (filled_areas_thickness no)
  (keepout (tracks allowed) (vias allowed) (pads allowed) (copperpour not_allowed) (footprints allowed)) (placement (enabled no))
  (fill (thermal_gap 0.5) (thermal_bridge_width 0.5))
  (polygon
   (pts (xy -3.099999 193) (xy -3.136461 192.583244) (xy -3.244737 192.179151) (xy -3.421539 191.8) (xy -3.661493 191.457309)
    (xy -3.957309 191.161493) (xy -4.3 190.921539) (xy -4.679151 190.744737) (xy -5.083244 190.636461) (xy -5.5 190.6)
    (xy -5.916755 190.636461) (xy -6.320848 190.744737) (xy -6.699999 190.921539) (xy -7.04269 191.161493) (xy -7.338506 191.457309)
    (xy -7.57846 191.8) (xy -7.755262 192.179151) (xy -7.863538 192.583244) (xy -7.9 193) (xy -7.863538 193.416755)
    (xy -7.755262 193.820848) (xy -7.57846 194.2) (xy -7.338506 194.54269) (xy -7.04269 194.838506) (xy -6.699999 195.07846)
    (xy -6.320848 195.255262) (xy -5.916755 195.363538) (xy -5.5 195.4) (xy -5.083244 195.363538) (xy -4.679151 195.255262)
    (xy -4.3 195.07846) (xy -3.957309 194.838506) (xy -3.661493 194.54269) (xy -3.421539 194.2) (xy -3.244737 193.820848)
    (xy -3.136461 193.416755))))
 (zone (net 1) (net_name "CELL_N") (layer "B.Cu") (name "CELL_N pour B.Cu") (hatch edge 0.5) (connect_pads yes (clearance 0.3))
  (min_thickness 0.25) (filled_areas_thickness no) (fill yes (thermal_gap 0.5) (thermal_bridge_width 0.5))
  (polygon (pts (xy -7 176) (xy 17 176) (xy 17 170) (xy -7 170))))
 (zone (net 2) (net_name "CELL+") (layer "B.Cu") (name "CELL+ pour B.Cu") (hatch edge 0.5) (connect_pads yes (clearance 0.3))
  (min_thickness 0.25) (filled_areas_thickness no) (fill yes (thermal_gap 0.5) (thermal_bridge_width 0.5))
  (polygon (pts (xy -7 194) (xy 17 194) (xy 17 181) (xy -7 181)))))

